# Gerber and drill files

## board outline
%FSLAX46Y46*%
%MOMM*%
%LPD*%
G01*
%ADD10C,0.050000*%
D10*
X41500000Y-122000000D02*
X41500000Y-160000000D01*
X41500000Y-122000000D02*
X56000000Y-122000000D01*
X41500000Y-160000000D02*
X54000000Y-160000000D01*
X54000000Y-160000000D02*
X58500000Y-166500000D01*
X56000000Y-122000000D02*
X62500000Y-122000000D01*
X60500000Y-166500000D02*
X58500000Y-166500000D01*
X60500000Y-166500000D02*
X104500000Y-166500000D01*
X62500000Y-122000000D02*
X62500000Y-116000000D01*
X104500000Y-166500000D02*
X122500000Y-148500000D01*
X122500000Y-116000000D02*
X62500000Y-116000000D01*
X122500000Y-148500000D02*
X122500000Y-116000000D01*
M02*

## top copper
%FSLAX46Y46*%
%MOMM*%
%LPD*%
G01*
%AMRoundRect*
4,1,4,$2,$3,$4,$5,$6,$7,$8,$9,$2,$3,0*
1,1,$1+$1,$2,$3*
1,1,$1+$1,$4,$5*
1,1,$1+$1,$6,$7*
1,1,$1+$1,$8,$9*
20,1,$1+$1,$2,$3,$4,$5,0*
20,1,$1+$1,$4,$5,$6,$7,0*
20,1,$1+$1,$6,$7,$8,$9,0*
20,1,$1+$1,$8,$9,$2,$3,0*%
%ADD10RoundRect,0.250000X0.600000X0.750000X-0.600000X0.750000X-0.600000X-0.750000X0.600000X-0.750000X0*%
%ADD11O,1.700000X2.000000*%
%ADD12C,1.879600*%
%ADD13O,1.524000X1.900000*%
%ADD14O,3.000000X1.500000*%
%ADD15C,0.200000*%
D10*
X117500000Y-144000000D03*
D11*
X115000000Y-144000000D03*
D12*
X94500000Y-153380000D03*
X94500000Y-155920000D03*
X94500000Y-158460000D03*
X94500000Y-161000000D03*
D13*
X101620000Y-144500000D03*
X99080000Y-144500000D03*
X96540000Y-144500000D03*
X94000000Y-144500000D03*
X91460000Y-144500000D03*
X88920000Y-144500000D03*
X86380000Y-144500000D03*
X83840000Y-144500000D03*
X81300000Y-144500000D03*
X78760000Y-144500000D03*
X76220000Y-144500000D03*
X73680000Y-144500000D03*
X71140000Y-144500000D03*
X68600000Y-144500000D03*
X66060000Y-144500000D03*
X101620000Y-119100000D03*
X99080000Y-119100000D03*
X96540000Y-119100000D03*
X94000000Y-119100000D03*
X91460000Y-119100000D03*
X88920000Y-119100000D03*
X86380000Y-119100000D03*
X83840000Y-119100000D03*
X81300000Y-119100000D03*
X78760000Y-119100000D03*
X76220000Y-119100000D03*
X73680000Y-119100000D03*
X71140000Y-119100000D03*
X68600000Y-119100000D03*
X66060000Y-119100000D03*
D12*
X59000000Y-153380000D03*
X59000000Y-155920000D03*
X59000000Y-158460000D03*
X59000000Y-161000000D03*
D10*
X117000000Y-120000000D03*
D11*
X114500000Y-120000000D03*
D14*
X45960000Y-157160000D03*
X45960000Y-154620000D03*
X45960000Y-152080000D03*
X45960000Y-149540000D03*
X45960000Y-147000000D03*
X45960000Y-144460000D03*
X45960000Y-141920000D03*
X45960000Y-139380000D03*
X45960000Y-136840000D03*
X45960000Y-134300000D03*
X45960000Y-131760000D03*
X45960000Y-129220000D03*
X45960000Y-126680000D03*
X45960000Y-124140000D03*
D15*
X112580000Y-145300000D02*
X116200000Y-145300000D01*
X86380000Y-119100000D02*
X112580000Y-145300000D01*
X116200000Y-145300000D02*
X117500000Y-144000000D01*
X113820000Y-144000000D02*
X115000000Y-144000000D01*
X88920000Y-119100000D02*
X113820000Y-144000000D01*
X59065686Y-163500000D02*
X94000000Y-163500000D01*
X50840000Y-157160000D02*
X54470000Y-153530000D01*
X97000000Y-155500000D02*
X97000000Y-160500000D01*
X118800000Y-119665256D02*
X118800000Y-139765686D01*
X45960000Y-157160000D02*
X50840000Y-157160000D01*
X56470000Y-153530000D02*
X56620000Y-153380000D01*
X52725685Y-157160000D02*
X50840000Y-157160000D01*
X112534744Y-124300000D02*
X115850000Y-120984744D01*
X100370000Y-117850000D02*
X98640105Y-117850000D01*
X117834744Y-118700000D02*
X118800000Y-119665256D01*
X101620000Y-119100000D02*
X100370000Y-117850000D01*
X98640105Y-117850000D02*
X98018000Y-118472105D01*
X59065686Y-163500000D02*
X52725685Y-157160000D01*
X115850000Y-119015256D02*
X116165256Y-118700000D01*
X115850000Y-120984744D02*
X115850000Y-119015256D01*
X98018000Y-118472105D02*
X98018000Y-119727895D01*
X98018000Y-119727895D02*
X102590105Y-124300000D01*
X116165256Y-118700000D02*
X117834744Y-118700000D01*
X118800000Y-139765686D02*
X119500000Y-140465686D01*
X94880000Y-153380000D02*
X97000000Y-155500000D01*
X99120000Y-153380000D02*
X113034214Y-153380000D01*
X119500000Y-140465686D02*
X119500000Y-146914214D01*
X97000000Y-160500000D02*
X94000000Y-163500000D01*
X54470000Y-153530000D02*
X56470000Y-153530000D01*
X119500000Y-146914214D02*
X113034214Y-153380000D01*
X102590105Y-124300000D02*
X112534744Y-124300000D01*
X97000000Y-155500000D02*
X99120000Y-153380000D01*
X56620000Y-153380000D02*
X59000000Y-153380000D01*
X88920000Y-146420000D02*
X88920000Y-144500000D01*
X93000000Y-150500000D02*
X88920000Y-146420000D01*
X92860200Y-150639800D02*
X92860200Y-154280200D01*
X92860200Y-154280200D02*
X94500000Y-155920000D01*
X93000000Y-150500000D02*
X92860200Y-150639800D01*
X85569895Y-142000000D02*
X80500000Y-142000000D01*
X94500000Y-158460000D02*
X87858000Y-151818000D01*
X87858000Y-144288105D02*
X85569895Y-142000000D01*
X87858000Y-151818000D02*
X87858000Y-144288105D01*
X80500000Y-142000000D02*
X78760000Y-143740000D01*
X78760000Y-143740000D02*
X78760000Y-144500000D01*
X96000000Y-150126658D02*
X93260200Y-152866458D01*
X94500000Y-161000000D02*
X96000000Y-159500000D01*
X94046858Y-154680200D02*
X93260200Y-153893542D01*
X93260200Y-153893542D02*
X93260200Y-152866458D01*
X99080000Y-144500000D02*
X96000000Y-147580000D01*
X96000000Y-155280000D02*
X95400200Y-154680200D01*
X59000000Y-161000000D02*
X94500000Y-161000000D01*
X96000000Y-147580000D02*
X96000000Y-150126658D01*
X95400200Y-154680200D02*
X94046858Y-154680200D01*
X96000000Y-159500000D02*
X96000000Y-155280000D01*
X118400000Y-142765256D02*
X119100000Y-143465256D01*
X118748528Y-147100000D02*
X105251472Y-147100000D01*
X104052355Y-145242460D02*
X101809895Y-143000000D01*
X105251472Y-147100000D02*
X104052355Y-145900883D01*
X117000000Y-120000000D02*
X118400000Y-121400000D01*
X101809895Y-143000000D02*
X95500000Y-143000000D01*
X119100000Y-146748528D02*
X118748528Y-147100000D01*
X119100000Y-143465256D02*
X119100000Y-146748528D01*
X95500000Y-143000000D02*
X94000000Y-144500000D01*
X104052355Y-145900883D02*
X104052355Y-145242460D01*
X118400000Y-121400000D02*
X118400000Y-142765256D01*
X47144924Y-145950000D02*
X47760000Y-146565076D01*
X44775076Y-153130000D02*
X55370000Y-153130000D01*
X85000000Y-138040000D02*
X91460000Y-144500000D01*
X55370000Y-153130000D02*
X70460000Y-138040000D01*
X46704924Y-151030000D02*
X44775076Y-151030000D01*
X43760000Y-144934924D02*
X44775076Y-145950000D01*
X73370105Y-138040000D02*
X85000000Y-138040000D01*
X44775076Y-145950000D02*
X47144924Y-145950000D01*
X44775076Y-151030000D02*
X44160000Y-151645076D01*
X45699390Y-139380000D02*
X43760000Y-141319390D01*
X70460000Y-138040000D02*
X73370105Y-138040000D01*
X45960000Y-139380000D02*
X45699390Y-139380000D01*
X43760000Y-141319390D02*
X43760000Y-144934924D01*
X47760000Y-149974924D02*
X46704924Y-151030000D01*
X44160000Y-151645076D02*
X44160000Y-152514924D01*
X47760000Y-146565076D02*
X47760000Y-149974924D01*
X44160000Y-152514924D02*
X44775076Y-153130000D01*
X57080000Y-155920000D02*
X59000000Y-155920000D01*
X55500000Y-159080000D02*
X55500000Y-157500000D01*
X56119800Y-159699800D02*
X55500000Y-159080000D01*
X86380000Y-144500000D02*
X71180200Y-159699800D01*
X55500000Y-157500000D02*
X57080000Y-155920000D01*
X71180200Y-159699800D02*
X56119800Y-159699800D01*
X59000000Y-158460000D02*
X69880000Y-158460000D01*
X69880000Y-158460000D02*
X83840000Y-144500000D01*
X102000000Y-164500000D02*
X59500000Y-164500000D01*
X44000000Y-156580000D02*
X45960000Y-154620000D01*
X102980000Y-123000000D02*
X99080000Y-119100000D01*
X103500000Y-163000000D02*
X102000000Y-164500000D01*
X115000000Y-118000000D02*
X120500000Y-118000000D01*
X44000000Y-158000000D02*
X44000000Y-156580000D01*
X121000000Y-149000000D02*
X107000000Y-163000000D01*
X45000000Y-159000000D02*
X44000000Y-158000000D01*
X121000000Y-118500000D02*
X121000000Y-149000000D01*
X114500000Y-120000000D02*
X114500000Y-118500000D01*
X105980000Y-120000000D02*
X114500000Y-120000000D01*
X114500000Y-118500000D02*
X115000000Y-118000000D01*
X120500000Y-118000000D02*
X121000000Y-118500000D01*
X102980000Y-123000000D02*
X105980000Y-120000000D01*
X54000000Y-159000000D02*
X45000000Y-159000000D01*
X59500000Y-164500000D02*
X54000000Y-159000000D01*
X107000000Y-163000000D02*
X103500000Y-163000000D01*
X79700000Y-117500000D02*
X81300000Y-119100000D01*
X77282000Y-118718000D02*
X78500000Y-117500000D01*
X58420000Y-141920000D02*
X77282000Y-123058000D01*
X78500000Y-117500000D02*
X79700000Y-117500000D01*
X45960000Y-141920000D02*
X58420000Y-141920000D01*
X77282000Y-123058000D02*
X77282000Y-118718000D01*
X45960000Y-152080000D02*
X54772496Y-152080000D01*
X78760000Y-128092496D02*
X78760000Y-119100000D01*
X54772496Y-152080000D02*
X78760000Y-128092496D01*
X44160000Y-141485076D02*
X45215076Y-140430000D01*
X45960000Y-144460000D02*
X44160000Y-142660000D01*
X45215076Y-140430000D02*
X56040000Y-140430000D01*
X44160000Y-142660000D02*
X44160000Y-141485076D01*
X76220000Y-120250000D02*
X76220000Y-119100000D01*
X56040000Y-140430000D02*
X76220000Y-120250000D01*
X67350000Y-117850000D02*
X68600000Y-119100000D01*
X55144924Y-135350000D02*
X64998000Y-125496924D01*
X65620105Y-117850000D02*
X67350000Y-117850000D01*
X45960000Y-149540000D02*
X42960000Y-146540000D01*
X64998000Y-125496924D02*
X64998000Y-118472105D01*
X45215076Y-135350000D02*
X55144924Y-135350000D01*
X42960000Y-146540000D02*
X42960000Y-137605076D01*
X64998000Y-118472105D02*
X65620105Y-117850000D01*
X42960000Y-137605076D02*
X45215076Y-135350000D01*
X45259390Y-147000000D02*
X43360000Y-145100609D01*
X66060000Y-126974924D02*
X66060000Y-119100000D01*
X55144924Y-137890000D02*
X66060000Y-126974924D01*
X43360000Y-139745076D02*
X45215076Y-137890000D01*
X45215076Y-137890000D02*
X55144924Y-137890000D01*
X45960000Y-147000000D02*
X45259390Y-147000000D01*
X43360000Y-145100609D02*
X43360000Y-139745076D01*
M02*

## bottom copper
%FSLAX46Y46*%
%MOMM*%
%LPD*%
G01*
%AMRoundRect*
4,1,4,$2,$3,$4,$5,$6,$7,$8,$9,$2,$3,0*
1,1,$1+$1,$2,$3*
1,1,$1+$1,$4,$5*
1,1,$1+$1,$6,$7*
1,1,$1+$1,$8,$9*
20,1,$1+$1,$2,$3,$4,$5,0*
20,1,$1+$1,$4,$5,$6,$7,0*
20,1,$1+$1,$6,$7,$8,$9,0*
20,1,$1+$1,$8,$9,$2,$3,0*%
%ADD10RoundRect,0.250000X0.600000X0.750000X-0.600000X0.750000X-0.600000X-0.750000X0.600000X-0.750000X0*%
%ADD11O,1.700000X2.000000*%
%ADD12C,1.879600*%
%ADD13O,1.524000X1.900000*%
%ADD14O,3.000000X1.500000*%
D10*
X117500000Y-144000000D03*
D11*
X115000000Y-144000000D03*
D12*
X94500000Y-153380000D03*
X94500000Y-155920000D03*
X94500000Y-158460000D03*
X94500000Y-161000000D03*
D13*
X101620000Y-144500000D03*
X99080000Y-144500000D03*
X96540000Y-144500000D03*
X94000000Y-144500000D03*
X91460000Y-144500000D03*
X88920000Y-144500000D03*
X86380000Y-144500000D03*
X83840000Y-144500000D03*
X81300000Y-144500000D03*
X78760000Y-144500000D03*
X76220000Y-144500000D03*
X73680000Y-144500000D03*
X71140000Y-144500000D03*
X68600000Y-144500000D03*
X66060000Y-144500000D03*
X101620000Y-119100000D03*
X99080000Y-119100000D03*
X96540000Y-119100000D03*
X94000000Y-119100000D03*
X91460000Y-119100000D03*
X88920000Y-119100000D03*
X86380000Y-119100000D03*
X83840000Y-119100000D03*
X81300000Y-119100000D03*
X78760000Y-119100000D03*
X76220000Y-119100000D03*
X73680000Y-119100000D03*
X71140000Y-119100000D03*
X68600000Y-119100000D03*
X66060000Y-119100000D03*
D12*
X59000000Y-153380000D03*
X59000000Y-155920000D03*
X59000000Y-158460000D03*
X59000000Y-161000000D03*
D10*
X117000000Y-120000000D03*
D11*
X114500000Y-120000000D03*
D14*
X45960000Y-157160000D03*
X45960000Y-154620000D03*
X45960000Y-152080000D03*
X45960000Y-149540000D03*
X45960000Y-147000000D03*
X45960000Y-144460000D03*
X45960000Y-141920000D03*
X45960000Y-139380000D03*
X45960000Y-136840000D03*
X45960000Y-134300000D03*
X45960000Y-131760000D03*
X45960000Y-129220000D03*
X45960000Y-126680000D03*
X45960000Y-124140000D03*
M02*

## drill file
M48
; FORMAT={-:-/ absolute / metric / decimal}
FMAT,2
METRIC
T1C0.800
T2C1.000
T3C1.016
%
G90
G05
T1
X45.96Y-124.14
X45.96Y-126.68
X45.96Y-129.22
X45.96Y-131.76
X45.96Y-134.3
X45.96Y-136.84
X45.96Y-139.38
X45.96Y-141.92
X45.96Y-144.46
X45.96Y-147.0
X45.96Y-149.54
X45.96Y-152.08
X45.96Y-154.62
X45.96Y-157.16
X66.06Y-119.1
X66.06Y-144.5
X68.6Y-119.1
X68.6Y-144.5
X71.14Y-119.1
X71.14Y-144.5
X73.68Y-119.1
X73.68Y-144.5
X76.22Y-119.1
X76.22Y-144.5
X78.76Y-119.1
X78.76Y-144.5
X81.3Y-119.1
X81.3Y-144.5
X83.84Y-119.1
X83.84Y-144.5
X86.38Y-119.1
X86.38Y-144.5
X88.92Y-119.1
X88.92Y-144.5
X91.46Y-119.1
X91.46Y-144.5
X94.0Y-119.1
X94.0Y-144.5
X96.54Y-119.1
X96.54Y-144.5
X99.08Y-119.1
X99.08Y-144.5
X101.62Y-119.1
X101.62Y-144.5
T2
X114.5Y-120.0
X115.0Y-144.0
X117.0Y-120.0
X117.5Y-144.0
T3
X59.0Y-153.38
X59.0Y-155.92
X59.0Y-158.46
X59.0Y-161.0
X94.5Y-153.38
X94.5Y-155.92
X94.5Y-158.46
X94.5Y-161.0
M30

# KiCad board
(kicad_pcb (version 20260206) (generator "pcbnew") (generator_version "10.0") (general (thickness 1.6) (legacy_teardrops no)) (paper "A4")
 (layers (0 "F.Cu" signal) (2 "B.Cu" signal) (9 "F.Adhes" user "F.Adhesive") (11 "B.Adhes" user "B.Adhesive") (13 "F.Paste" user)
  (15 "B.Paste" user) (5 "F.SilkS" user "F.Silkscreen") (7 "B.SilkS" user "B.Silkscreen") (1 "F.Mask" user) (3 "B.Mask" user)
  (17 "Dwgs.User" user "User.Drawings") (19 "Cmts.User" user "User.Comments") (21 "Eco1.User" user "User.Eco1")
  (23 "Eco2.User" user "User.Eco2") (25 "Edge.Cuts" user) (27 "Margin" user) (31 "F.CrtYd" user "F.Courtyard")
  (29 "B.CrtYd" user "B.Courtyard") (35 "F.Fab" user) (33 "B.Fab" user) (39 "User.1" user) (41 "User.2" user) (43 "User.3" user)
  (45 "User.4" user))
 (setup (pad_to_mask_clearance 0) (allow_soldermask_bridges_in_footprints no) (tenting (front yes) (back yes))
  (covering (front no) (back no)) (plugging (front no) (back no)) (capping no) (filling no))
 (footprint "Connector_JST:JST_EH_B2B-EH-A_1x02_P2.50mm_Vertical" (layer "F.Cu") (at 117.5 144 180)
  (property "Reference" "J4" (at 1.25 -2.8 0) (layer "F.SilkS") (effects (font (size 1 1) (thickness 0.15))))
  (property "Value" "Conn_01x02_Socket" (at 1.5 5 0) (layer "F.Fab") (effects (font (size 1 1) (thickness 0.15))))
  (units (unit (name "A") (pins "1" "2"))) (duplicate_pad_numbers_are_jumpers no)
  (pad "1" thru_hole roundrect (at 0 0 180) (size 1.7 2) (drill 1) (layers "*.Cu" "*.Mask") (remove_unused_layers no)
   (roundrect_rratio 0.147059) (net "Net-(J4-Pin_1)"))
  (pad "2" thru_hole oval (at 2.5 0 180) (size 1.7 2) (drill 1) (layers "*.Cu" "*.Mask") (remove_unused_layers no) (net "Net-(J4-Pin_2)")))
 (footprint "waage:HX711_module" (layer "F.Cu") (at 106.5 157.18 180)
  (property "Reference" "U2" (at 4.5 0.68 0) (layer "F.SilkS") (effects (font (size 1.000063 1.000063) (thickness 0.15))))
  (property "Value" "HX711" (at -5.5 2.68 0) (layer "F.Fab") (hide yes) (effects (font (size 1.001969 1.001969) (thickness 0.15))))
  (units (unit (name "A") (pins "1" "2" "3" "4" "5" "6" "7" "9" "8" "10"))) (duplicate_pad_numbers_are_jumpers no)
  (pad "7" thru_hole circle (at 12 3.8 180) (size 1.8796 1.8796) (drill 1.016) (layers "*.Cu" "*.Mask") (remove_unused_layers no)
   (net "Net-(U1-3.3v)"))
  (pad "8" thru_hole circle (at 12 1.26 180) (size 1.8796 1.8796) (drill 1.016) (layers "*.Cu" "*.Mask") (remove_unused_layers no)
   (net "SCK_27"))
  (pad "9" thru_hole circle (at 12 -1.28 180) (size 1.8796 1.8796) (drill 1.016) (layers "*.Cu" "*.Mask") (remove_unused_layers no)
   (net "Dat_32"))
  (pad "10" thru_hole circle (at 12 -3.82 180) (size 1.8796 1.8796) (drill 1.016) (layers "*.Cu" "*.Mask") (remove_unused_layers no)
   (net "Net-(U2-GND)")))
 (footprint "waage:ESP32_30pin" (layer "F.Cu") (at 84.600187 132.57246 90)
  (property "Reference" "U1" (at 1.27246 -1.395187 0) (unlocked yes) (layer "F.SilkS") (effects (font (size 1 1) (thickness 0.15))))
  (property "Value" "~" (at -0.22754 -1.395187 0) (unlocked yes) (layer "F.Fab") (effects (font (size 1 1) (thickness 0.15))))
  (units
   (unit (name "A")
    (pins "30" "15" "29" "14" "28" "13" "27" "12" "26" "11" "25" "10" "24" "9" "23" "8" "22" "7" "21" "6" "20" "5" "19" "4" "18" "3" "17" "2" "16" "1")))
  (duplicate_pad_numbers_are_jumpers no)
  (pad "1" thru_hole oval (at -11.92754 17.019813) (size 1.524 1.9) (drill 0.8) (layers "*.Cu" "*.Mask") (remove_unused_layers no)
   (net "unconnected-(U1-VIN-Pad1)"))
  (pad "2" thru_hole oval (at -11.92754 14.479813) (size 1.524 1.9) (drill 0.8) (layers "*.Cu" "*.Mask") (remove_unused_layers no)
   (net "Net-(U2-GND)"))
  (pad "3" thru_hole oval (at -11.92754 11.939813) (size 1.524 1.9) (drill 0.8) (layers "*.Cu" "*.Mask") (remove_unused_layers no)
   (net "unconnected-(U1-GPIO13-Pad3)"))
  (pad "4" thru_hole oval (at -11.92754 9.399813) (size 1.524 1.9) (drill 0.8) (layers "*.Cu" "*.Mask") (remove_unused_layers no)
   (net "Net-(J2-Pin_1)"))
  (pad "5" thru_hole oval (at -11.92754 6.859813) (size 1.524 1.9) (drill 0.8) (layers "*.Cu" "*.Mask") (remove_unused_layers no)
   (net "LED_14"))
  (pad "6" thru_hole oval (at -11.92754 4.319813) (size 1.524 1.9) (drill 0.8) (layers "*.Cu" "*.Mask") (remove_unused_layers no)
   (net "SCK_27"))
  (pad "7" thru_hole oval (at -11.92754 1.779813) (size 1.524 1.9) (drill 0.8) (layers "*.Cu" "*.Mask") (remove_unused_layers no)
   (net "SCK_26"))
  (pad "8" thru_hole oval (at -11.92754 -0.760187) (size 1.524 1.9) (drill 0.8) (layers "*.Cu" "*.Mask") (remove_unused_layers no)
   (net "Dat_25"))
  (pad "9" thru_hole oval (at -11.92754 -3.300187) (size 1.524 1.9) (drill 0.8) (layers "*.Cu" "*.Mask") (remove_unused_layers no)
   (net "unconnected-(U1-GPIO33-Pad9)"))
  (pad "10" thru_hole oval (at -11.92754 -5.840187) (size 1.524 1.9) (drill 0.8) (layers "*.Cu" "*.Mask") (remove_unused_layers no)
   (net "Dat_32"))
  (pad "11" thru_hole oval (at -11.92754 -8.380187) (size 1.524 1.9) (drill 0.8) (layers "*.Cu" "*.Mask") (remove_unused_layers no)
   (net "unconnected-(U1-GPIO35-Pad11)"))
  (pad "12" thru_hole oval (at -11.92754 -10.920187) (size 1.524 1.9) (drill 0.8) (layers "*.Cu" "*.Mask") (remove_unused_layers no)
   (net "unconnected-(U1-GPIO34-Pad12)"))
  (pad "13" thru_hole oval (at -11.92754 -13.460187) (size 1.524 1.9) (drill 0.8) (layers "*.Cu" "*.Mask") (remove_unused_layers no)
   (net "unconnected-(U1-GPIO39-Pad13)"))
  (pad "14" thru_hole oval (at -11.92754 -16.000187) (size 1.524 1.9) (drill 0.8) (layers "*.Cu" "*.Mask") (remove_unused_layers no)
   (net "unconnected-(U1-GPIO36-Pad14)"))
  (pad "15" thru_hole oval (at -11.92754 -18.540187) (size 1.524 1.9) (drill 0.8) (layers "*.Cu" "*.Mask") (remove_unused_layers no)
   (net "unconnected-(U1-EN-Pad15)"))
  (pad "16" thru_hole oval (at 13.47246 17.019813) (size 1.524 1.9) (drill 0.8) (layers "*.Cu" "*.Mask") (remove_unused_layers no)
   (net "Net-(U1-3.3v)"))
  (pad "17" thru_hole oval (at 13.47246 14.479813) (size 1.524 1.9) (drill 0.8) (layers "*.Cu" "*.Mask") (remove_unused_layers no)
   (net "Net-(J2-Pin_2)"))
  (pad "18" thru_hole oval (at 13.47246 11.939813) (size 1.524 1.9) (drill 0.8) (layers "*.Cu" "*.Mask") (remove_unused_layers no)
   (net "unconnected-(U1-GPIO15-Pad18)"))
  (pad "19" thru_hole oval (at 13.47246 9.399813) (size 1.524 1.9) (drill 0.8) (layers "*.Cu" "*.Mask") (remove_unused_layers no)
   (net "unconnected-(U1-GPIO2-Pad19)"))
  (pad "20" thru_hole oval (at 13.47246 6.859813) (size 1.524 1.9) (drill 0.8) (layers "*.Cu" "*.Mask" "Dwgs.User")
   (remove_unused_layers no) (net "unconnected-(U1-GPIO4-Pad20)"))
  (pad "21" thru_hole oval (at 13.47246 4.319813) (size 1.524 1.9) (drill 0.8) (layers "*.Cu" "*.Mask") (remove_unused_layers no)
   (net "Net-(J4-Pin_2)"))
  (pad "22" thru_hole oval (at 13.47246 1.779813) (size 1.524 1.9) (drill 0.8) (layers "*.Cu" "*.Mask") (remove_unused_layers no)
   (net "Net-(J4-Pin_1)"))
  (pad "23" thru_hole oval (at 13.47246 -0.760187) (size 1.524 1.9) (drill 0.8) (layers "*.Cu" "*.Mask") (remove_unused_layers no)
   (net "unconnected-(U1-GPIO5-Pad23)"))
  (pad "24" thru_hole oval (at 13.47246 -3.300187) (size 1.524 1.9) (drill 0.8) (layers "*.Cu" "*.Mask") (remove_unused_layers no)
   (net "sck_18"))
  (pad "25" thru_hole oval (at 13.47246 -5.840187) (size 1.524 1.9) (drill 0.8) (layers "*.Cu" "*.Mask") (remove_unused_layers no)
   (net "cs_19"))
  (pad "26" thru_hole oval (at 13.47246 -8.380187) (size 1.524 1.9) (drill 0.8) (layers "*.Cu" "*.Mask") (remove_unused_layers no)
   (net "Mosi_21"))
  (pad "27" thru_hole oval (at 13.47246 -10.920187) (size 1.524 1.9) (drill 0.8) (layers "*.Cu" "*.Mask") (remove_unused_layers no)
   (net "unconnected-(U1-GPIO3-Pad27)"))
  (pad "28" thru_hole oval (at 13.47246 -13.460187) (size 1.524 1.9) (drill 0.8) (layers "*.Cu" "*.Mask") (remove_unused_layers no)
   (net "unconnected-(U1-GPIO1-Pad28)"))
  (pad "29" thru_hole oval (at 13.47246 -16.000187) (size 1.524 1.9) (drill 0.8) (layers "*.Cu" "*.Mask") (remove_unused_layers no)
   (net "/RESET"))
  (pad "30" thru_hole oval (at 13.47246 -18.540187) (size 1.524 1.9) (drill 0.8) (layers "*.Cu" "*.Mask") (remove_unused_layers no)
   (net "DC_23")))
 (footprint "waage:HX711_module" (layer "F.Cu") (at 71 157.18 180)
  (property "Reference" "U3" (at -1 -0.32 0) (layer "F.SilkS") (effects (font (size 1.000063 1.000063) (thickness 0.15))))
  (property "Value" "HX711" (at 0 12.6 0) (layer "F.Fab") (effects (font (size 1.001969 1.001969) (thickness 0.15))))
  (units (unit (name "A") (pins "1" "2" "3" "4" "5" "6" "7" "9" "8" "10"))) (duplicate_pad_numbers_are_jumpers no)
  (pad "7" thru_hole circle (at 12 3.8 180) (size 1.8796 1.8796) (drill 1.016) (layers "*.Cu" "*.Mask") (remove_unused_layers no)
   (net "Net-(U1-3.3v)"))
  (pad "8" thru_hole circle (at 12 1.26 180) (size 1.8796 1.8796) (drill 1.016) (layers "*.Cu" "*.Mask") (remove_unused_layers no)
   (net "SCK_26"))
  (pad "9" thru_hole circle (at 12 -1.28 180) (size 1.8796 1.8796) (drill 1.016) (layers "*.Cu" "*.Mask") (remove_unused_layers no)
   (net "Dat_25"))
  (pad "10" thru_hole circle (at 12 -3.82 180) (size 1.8796 1.8796) (drill 1.016) (layers "*.Cu" "*.Mask") (remove_unused_layers no)
   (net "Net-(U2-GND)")))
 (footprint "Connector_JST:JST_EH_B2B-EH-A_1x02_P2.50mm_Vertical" (layer "F.Cu") (at 117 120 180)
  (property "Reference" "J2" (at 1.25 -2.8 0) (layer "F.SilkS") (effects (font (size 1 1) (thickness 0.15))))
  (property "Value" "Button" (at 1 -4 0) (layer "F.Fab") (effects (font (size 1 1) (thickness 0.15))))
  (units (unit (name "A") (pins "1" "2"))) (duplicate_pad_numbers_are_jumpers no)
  (pad "1" thru_hole roundrect (at 0 0 180) (size 1.7 2) (drill 1) (layers "*.Cu" "*.Mask") (remove_unused_layers no)
   (roundrect_rratio 0.147059) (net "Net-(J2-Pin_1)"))
  (pad "2" thru_hole oval (at 2.5 0 180) (size 1.7 2) (drill 1) (layers "*.Cu" "*.Mask") (remove_unused_layers no) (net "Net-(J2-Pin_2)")))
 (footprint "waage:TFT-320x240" (layer "B.Cu") (at 45.96 140.65 90)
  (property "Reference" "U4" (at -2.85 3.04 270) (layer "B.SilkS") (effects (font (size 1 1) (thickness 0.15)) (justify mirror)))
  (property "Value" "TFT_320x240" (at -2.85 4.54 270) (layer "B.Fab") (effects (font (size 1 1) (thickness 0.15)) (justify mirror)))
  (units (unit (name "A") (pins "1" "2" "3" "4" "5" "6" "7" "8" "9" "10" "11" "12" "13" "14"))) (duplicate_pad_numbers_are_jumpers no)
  (pad "1" thru_hole oval (at -16.51 0 90) (size 1.5 3) (drill 0.8) (layers "*.Cu" "*.Mask") (remove_unused_layers no) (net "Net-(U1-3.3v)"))
  (pad "2" thru_hole oval (at -13.97 0 90) (size 1.5 3) (drill 0.8) (layers "*.Cu" "*.Mask") (remove_unused_layers no)
   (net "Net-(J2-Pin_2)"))
  (pad "3" thru_hole oval (at -11.43 0 90) (size 1.5 3) (drill 0.8) (layers "*.Cu" "*.Mask") (remove_unused_layers no) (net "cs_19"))
  (pad "4" thru_hole oval (at -8.89 0 90) (size 1.5 3) (drill 0.8) (layers "*.Cu" "*.Mask") (remove_unused_layers no) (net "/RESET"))
  (pad "5" thru_hole oval (at -6.35 0 90) (size 1.5 3) (drill 0.8) (layers "*.Cu" "*.Mask") (remove_unused_layers no) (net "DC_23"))
  (pad "6" thru_hole oval (at -3.81 0 90) (size 1.5 3) (drill 0.8) (layers "*.Cu" "*.Mask") (remove_unused_layers no) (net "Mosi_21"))
  (pad "7" thru_hole oval (at -1.27 0 90) (size 1.5 3) (drill 0.8) (layers "*.Cu" "*.Mask") (remove_unused_layers no) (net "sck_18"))
  (pad "8" thru_hole oval (at 1.27 0 90) (size 1.5 3) (drill 0.8) (layers "*.Cu" "*.Mask") (remove_unused_layers no) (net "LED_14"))
  (pad "9" thru_hole oval (at 3.81 0 90) (size 1.5 3) (drill 0.8) (layers "*.Cu" "*.Mask") (remove_unused_layers no)
   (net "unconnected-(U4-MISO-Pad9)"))
  (pad "10" thru_hole oval (at 6.35 0 90) (size 1.5 3) (drill 0.8) (layers "*.Cu" "*.Mask") (remove_unused_layers no)
   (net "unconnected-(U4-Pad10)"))
  (pad "11" thru_hole oval (at 8.89 0 90) (size 1.5 3) (drill 0.8) (layers "*.Cu" "*.Mask") (remove_unused_layers no)
   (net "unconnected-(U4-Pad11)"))
  (pad "12" thru_hole oval (at 11.43 0 90) (size 1.5 3) (drill 0.8) (layers "*.Cu" "*.Mask") (remove_unused_layers no)
   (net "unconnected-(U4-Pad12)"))
  (pad "13" thru_hole oval (at 13.97 0 90) (size 1.5 3) (drill 0.8) (layers "*.Cu" "*.Mask") (remove_unused_layers no)
   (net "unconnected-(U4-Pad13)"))
  (pad "14" thru_hole oval (at 16.51 0 90) (size 1.5 3) (drill 0.8) (layers "*.Cu" "*.Mask") (remove_unused_layers no)
   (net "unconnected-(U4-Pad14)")))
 (gr_line (start 41.5 122) (end 41.5 160) (stroke (width 0.05) (type default)) (layer "Edge.Cuts"))
 (gr_line (start 41.5 122) (end 56 122) (stroke (width 0.05) (type default)) (layer "Edge.Cuts"))
 (gr_line (start 41.5 160) (end 54 160) (stroke (width 0.05) (type default)) (layer "Edge.Cuts"))
 (gr_line (start 54 160) (end 58.5 166.5) (stroke (width 0.05) (type default)) (layer "Edge.Cuts"))
 (gr_line (start 56 122) (end 62.5 122) (stroke (width 0.05) (type default)) (layer "Edge.Cuts"))
 (gr_line (start 60.5 166.5) (end 58.5 166.5) (stroke (width 0.05) (type default)) (layer "Edge.Cuts"))
 (gr_line (start 60.5 166.5) (end 104.5 166.5) (stroke (width 0.05) (type default)) (layer "Edge.Cuts"))
 (gr_line (start 62.5 122) (end 62.5 116) (stroke (width 0.05) (type default)) (layer "Edge.Cuts"))
 (gr_line (start 104.5 166.5) (end 122.5 148.5) (stroke (width 0.05) (type default)) (layer "Edge.Cuts"))
 (gr_line (start 122.5 116) (end 62.5 116) (stroke (width 0.05) (type default)) (layer "Edge.Cuts"))
 (gr_line (start 122.5 148.5) (end 122.5 116) (stroke (width 0.05) (type default)) (layer "Edge.Cuts"))
 (segment (start 112.58 145.3) (end 116.2 145.3) (width 0.2) (layer "F.Cu") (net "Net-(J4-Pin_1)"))
 (segment (start 86.38 119.1) (end 112.58 145.3) (width 0.2) (layer "F.Cu") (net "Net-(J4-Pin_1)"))
 (segment (start 116.2 145.3) (end 117.5 144) (width 0.2) (layer "F.Cu") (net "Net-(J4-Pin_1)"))
 (segment (start 113.82 144) (end 115 144) (width 0.2) (layer "F.Cu") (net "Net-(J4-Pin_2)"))
 (segment (start 88.92 119.1) (end 113.82 144) (width 0.2) (layer "F.Cu") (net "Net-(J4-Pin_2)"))
 (segment (start 59.065686 163.5) (end 94 163.5) (width 0.2) (layer "F.Cu") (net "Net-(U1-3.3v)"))
 (segment (start 50.84 157.16) (end 54.47 153.53) (width 0.2) (layer "F.Cu") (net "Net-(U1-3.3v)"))
 (segment (start 97 155.5) (end 97 160.5) (width 0.2) (layer "F.Cu") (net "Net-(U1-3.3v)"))
 (segment (start 118.8 119.665256) (end 118.8 139.765686) (width 0.2) (layer "F.Cu") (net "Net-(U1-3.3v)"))
 (segment (start 45.96 157.16) (end 50.84 157.16) (width 0.2) (layer "F.Cu") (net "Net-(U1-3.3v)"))
 (segment (start 56.47 153.53) (end 56.62 153.38) (width 0.2) (layer "F.Cu") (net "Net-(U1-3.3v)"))
 (segment (start 52.725685 157.16) (end 50.84 157.16) (width 0.2) (layer "F.Cu") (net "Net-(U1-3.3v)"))
 (segment (start 112.534744 124.3) (end 115.85 120.984744) (width 0.2) (layer "F.Cu") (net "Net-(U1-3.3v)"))
 (segment (start 100.37 117.85) (end 98.640105 117.85) (width 0.2) (layer "F.Cu") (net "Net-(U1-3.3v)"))
 (segment (start 117.834744 118.7) (end 118.8 119.665256) (width 0.2) (layer "F.Cu") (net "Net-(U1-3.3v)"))
 (segment (start 101.62 119.1) (end 100.37 117.85) (width 0.2) (layer "F.Cu") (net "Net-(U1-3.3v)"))
 (segment (start 98.640105 117.85) (end 98.018 118.472105) (width 0.2) (layer "F.Cu") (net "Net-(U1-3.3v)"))
 (segment (start 59.065686 163.5) (end 52.725685 157.16) (width 0.2) (layer "F.Cu") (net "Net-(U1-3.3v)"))
 (segment (start 115.85 119.015256) (end 116.165256 118.7) (width 0.2) (layer "F.Cu") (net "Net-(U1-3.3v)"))
 (segment (start 115.85 120.984744) (end 115.85 119.015256) (width 0.2) (layer "F.Cu") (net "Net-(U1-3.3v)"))
 (segment (start 98.018 118.472105) (end 98.018 119.727895) (width 0.2) (layer "F.Cu") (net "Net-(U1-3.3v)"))
 (segment (start 98.018 119.727895) (end 102.590105 124.3) (width 0.2) (layer "F.Cu") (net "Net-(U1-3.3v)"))
 (segment (start 116.165256 118.7) (end 117.834744 118.7) (width 0.2) (layer "F.Cu") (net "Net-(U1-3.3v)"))
 (segment (start 118.8 139.765686) (end 119.5 140.465686) (width 0.2) (layer "F.Cu") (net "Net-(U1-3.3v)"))
 (segment (start 94.88 153.38) (end 97 155.5) (width 0.2) (layer "F.Cu") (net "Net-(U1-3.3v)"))
 (segment (start 99.12 153.38) (end 113.034214 153.38) (width 0.2) (layer "F.Cu") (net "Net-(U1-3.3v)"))
 (segment (start 119.5 140.465686) (end 119.5 146.914214) (width 0.2) (layer "F.Cu") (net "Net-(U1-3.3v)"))
 (segment (start 97 160.5) (end 94 163.5) (width 0.2) (layer "F.Cu") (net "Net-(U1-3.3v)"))
 (segment (start 54.47 153.53) (end 56.47 153.53) (width 0.2) (layer "F.Cu") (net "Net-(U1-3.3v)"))
 (segment (start 119.5 146.914214) (end 113.034214 153.38) (width 0.2) (layer "F.Cu") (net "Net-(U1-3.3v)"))
 (segment (start 102.590105 124.3) (end 112.534744 124.3) (width 0.2) (layer "F.Cu") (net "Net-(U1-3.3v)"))
 (segment (start 97 155.5) (end 99.12 153.38) (width 0.2) (layer "F.Cu") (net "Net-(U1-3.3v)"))
 (segment (start 56.62 153.38) (end 59 153.38) (width 0.2) (layer "F.Cu") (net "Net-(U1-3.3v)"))
 (segment (start 88.92 146.42) (end 88.92 144.5) (width 0.2) (layer "F.Cu") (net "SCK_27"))
 (segment (start 93 150.5) (end 88.92 146.42) (width 0.2) (layer "F.Cu") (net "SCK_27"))
 (segment (start 92.8602 150.6398) (end 92.8602 154.2802) (width 0.2) (layer "F.Cu") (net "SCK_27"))
 (segment (start 92.8602 154.2802) (end 94.5 155.92) (width 0.2) (layer "F.Cu") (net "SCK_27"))
 (segment (start 93 150.5) (end 92.8602 150.6398) (width 0.2) (layer "F.Cu") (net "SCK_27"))
 (segment (start 85.569895 142) (end 80.5 142) (width 0.2) (layer "F.Cu") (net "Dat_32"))
 (segment (start 94.5 158.46) (end 87.858 151.818) (width 0.2) (layer "F.Cu") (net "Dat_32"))
 (segment (start 87.858 144.288105) (end 85.569895 142) (width 0.2) (layer "F.Cu") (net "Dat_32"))
 (segment (start 87.858 151.818) (end 87.858 144.288105) (width 0.2) (layer "F.Cu") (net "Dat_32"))
 (segment (start 80.5 142) (end 78.76 143.74) (width 0.2) (layer "F.Cu") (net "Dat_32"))
 (segment (start 78.76 143.74) (end 78.76 144.5) (width 0.2) (layer "F.Cu") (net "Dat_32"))
 (segment (start 96 150.126658) (end 93.2602 152.866458) (width 0.2) (layer "F.Cu") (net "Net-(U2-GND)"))
 (segment (start 94.5 161) (end 96 159.5) (width 0.2) (layer "F.Cu") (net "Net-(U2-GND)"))
 (segment (start 94.046858 154.6802) (end 93.2602 153.893542) (width 0.2) (layer "F.Cu") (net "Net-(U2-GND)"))
 (segment (start 93.2602 153.893542) (end 93.2602 152.866458) (width 0.2) (layer "F.Cu") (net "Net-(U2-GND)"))
 (segment (start 99.08 144.5) (end 96 147.58) (width 0.2) (layer "F.Cu") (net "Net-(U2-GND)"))
 (segment (start 96 155.28) (end 95.4002 154.6802) (width 0.2) (layer "F.Cu") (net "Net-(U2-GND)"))
 (segment (start 59 161) (end 94.5 161) (width 0.2) (layer "F.Cu") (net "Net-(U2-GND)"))
 (segment (start 96 147.58) (end 96 150.126658) (width 0.2) (layer "F.Cu") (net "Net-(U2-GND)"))
 (segment (start 95.4002 154.6802) (end 94.046858 154.6802) (width 0.2) (layer "F.Cu") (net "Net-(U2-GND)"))
 (segment (start 96 159.5) (end 96 155.28) (width 0.2) (layer "F.Cu") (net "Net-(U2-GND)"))
 (segment (start 118.4 142.765256) (end 119.1 143.465256) (width 0.2) (layer "F.Cu") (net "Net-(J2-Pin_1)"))
 (segment (start 118.748528 147.1) (end 105.251472 147.1) (width 0.2) (layer "F.Cu") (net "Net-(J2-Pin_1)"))
 (segment (start 104.052355 145.24246) (end 101.809895 143) (width 0.2) (layer "F.Cu") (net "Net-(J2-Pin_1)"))
 (segment (start 105.251472 147.1) (end 104.052355 145.900883) (width 0.2) (layer "F.Cu") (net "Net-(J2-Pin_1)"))
 (segment (start 117 120) (end 118.4 121.4) (width 0.2) (layer "F.Cu") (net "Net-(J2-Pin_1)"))
 (segment (start 101.809895 143) (end 95.5 143) (width 0.2) (layer "F.Cu") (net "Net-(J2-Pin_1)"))
 (segment (start 119.1 146.748528) (end 118.748528 147.1) (width 0.2) (layer "F.Cu") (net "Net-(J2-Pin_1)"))
 (segment (start 119.1 143.465256) (end 119.1 146.748528) (width 0.2) (layer "F.Cu") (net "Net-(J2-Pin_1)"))
 (segment (start 95.5 143) (end 94 144.5) (width 0.2) (layer "F.Cu") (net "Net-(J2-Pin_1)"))
 (segment (start 104.052355 145.900883) (end 104.052355 145.24246) (width 0.2) (layer "F.Cu") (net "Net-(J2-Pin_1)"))
 (segment (start 118.4 121.4) (end 118.4 142.765256) (width 0.2) (layer "F.Cu") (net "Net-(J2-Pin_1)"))
 (segment (start 47.144924 145.95) (end 47.76 146.565076) (width 0.2) (layer "F.Cu") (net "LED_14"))
 (segment (start 44.775076 153.13) (end 55.37 153.13) (width 0.2) (layer "F.Cu") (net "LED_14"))
 (segment (start 85 138.04) (end 91.46 144.5) (width 0.2) (layer "F.Cu") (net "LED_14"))
 (segment (start 55.37 153.13) (end 70.46 138.04) (width 0.2) (layer "F.Cu") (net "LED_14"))
 (segment (start 46.704924 151.03) (end 44.775076 151.03) (width 0.2) (layer "F.Cu") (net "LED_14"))
 (segment (start 43.76 144.934924) (end 44.775076 145.95) (width 0.2) (layer "F.Cu") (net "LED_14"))
 (segment (start 73.370105 138.04) (end 85 138.04) (width 0.2) (layer "F.Cu") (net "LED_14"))
 (segment (start 44.775076 145.95) (end 47.144924 145.95) (width 0.2) (layer "F.Cu") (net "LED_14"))
 (segment (start 44.775076 151.03) (end 44.16 151.645076) (width 0.2) (layer "F.Cu") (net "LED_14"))
 (segment (start 45.69939 139.38) (end 43.76 141.31939) (width 0.2) (layer "F.Cu") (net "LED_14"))
 (segment (start 70.46 138.04) (end 73.370105 138.04) (width 0.2) (layer "F.Cu") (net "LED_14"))
 (segment (start 45.96 139.38) (end 45.69939 139.38) (width 0.2) (layer "F.Cu") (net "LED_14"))
 (segment (start 43.76 141.31939) (end 43.76 144.934924) (width 0.2) (layer "F.Cu") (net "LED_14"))
 (segment (start 47.76 149.974924) (end 46.704924 151.03) (width 0.2) (layer "F.Cu") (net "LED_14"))
 (segment (start 44.16 151.645076) (end 44.16 152.514924) (width 0.2) (layer "F.Cu") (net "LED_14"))
 (segment (start 47.76 146.565076) (end 47.76 149.974924) (width 0.2) (layer "F.Cu") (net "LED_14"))
 (segment (start 44.16 152.514924) (end 44.775076 153.13) (width 0.2) (layer "F.Cu") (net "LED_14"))
 (segment (start 57.08 155.92) (end 59 155.92) (width 0.2) (layer "F.Cu") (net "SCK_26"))
 (segment (start 55.5 159.08) (end 55.5 157.5) (width 0.2) (layer "F.Cu") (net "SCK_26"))
 (segment (start 56.1198 159.6998) (end 55.5 159.08) (width 0.2) (layer "F.Cu") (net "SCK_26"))
 (segment (start 86.38 144.5) (end 71.1802 159.6998) (width 0.2) (layer "F.Cu") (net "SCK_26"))
 (segment (start 55.5 157.5) (end 57.08 155.92) (width 0.2) (layer "F.Cu") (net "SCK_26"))
 (segment (start 71.1802 159.6998) (end 56.1198 159.6998) (width 0.2) (layer "F.Cu") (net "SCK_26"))
 (segment (start 59 158.46) (end 69.88 158.46) (width 0.2) (layer "F.Cu") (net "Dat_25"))
 (segment (start 69.88 158.46) (end 83.84 144.5) (width 0.2) (layer "F.Cu") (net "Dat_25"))
 (segment (start 102 164.5) (end 59.5 164.5) (width 0.2) (layer "F.Cu") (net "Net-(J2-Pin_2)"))
 (segment (start 44 156.58) (end 45.96 154.62) (width 0.2) (layer "F.Cu") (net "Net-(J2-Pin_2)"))
 (segment (start 102.98 123) (end 99.08 119.1) (width 0.2) (layer "F.Cu") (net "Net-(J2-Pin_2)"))
 (segment (start 103.5 163) (end 102 164.5) (width 0.2) (layer "F.Cu") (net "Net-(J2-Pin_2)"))
 (segment (start 115 118) (end 120.5 118) (width 0.2) (layer "F.Cu") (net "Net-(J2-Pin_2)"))
 (segment (start 44 158) (end 44 156.58) (width 0.2) (layer "F.Cu") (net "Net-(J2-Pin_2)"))
 (segment (start 121 149) (end 107 163) (width 0.2) (layer "F.Cu") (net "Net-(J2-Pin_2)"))
 (segment (start 45 159) (end 44 158) (width 0.2) (layer "F.Cu") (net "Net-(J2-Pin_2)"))
 (segment (start 121 118.5) (end 121 149) (width 0.2) (layer "F.Cu") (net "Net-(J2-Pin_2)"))
 (segment (start 114.5 120) (end 114.5 118.5) (width 0.2) (layer "F.Cu") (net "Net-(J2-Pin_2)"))
 (segment (start 105.98 120) (end 114.5 120) (width 0.2) (layer "F.Cu") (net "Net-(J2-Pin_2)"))
 (segment (start 114.5 118.5) (end 115 118) (width 0.2) (layer "F.Cu") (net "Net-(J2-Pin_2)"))
 (segment (start 120.5 118) (end 121 118.5) (width 0.2) (layer "F.Cu") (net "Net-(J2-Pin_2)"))
 (segment (start 102.98 123) (end 105.98 120) (width 0.2) (layer "F.Cu") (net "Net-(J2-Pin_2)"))
 (segment (start 54 159) (end 45 159) (width 0.2) (layer "F.Cu") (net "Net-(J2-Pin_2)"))
 (segment (start 59.5 164.5) (end 54 159) (width 0.2) (layer "F.Cu") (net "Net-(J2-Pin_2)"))
 (segment (start 107 163) (end 103.5 163) (width 0.2) (layer "F.Cu") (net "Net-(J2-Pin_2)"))
 (segment (start 79.7 117.5) (end 81.3 119.1) (width 0.2) (layer "F.Cu") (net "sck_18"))
 (segment (start 77.282 118.718) (end 78.5 117.5) (width 0.2) (layer "F.Cu") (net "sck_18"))
 (segment (start 58.42 141.92) (end 77.282 123.058) (width 0.2) (layer "F.Cu") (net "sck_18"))
 (segment (start 78.5 117.5) (end 79.7 117.5) (width 0.2) (layer "F.Cu") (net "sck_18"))
 (segment (start 45.96 141.92) (end 58.42 141.92) (width 0.2) (layer "F.Cu") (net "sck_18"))
 (segment (start 77.282 123.058) (end 77.282 118.718) (width 0.2) (layer "F.Cu") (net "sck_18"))
 (segment (start 45.96 152.08) (end 54.772496 152.08) (width 0.2) (layer "F.Cu") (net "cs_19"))
 (segment (start 78.76 128.092496) (end 78.76 119.1) (width 0.2) (layer "F.Cu") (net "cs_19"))
 (segment (start 54.772496 152.08) (end 78.76 128.092496) (width 0.2) (layer "F.Cu") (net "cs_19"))
 (segment (start 44.16 141.485076) (end 45.215076 140.43) (width 0.2) (layer "F.Cu") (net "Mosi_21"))
 (segment (start 45.96 144.46) (end 44.16 142.66) (width 0.2) (layer "F.Cu") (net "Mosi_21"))
 (segment (start 45.215076 140.43) (end 56.04 140.43) (width 0.2) (layer "F.Cu") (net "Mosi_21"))
 (segment (start 44.16 142.66) (end 44.16 141.485076) (width 0.2) (layer "F.Cu") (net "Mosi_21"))
 (segment (start 76.22 120.25) (end 76.22 119.1) (width 0.2) (layer "F.Cu") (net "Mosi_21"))
 (segment (start 56.04 140.43) (end 76.22 120.25) (width 0.2) (layer "F.Cu") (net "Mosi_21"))
 (segment (start 67.35 117.85) (end 68.6 119.1) (width 0.2) (layer "F.Cu") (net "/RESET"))
 (segment (start 55.144924 135.35) (end 64.998 125.496924) (width 0.2) (layer "F.Cu") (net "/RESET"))
 (segment (start 65.620105 117.85) (end 67.35 117.85) (width 0.2) (layer "F.Cu") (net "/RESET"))
 (segment (start 45.96 149.54) (end 42.96 146.54) (width 0.2) (layer "F.Cu") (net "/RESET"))
 (segment (start 64.998 125.496924) (end 64.998 118.472105) (width 0.2) (layer "F.Cu") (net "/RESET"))
 (segment (start 45.215076 135.35) (end 55.144924 135.35) (width 0.2) (layer "F.Cu") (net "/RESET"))
 (segment (start 42.96 146.54) (end 42.96 137.605076) (width 0.2) (layer "F.Cu") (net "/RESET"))
 (segment (start 64.998 118.472105) (end 65.620105 117.85) (width 0.2) (layer "F.Cu") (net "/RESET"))
 (segment (start 42.96 137.605076) (end 45.215076 135.35) (width 0.2) (layer "F.Cu") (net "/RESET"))
 (segment (start 45.25939 147) (end 43.36 145.100609) (width 0.2) (layer "F.Cu") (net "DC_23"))
 (segment (start 66.06 126.974924) (end 66.06 119.1) (width 0.2) (layer "F.Cu") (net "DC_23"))
 (segment (start 55.144924 137.89) (end 66.06 126.974924) (width 0.2) (layer "F.Cu") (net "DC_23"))
 (segment (start 43.36 139.745076) (end 45.215076 137.89) (width 0.2) (layer "F.Cu") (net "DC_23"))
 (segment (start 45.215076 137.89) (end 55.144924 137.89) (width 0.2) (layer "F.Cu") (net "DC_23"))
 (segment (start 45.96 147) (end 45.25939 147) (width 0.2) (layer "F.Cu") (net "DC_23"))
 (segment (start 43.36 145.100609) (end 43.36 139.745076) (width 0.2) (layer "F.Cu") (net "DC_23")))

